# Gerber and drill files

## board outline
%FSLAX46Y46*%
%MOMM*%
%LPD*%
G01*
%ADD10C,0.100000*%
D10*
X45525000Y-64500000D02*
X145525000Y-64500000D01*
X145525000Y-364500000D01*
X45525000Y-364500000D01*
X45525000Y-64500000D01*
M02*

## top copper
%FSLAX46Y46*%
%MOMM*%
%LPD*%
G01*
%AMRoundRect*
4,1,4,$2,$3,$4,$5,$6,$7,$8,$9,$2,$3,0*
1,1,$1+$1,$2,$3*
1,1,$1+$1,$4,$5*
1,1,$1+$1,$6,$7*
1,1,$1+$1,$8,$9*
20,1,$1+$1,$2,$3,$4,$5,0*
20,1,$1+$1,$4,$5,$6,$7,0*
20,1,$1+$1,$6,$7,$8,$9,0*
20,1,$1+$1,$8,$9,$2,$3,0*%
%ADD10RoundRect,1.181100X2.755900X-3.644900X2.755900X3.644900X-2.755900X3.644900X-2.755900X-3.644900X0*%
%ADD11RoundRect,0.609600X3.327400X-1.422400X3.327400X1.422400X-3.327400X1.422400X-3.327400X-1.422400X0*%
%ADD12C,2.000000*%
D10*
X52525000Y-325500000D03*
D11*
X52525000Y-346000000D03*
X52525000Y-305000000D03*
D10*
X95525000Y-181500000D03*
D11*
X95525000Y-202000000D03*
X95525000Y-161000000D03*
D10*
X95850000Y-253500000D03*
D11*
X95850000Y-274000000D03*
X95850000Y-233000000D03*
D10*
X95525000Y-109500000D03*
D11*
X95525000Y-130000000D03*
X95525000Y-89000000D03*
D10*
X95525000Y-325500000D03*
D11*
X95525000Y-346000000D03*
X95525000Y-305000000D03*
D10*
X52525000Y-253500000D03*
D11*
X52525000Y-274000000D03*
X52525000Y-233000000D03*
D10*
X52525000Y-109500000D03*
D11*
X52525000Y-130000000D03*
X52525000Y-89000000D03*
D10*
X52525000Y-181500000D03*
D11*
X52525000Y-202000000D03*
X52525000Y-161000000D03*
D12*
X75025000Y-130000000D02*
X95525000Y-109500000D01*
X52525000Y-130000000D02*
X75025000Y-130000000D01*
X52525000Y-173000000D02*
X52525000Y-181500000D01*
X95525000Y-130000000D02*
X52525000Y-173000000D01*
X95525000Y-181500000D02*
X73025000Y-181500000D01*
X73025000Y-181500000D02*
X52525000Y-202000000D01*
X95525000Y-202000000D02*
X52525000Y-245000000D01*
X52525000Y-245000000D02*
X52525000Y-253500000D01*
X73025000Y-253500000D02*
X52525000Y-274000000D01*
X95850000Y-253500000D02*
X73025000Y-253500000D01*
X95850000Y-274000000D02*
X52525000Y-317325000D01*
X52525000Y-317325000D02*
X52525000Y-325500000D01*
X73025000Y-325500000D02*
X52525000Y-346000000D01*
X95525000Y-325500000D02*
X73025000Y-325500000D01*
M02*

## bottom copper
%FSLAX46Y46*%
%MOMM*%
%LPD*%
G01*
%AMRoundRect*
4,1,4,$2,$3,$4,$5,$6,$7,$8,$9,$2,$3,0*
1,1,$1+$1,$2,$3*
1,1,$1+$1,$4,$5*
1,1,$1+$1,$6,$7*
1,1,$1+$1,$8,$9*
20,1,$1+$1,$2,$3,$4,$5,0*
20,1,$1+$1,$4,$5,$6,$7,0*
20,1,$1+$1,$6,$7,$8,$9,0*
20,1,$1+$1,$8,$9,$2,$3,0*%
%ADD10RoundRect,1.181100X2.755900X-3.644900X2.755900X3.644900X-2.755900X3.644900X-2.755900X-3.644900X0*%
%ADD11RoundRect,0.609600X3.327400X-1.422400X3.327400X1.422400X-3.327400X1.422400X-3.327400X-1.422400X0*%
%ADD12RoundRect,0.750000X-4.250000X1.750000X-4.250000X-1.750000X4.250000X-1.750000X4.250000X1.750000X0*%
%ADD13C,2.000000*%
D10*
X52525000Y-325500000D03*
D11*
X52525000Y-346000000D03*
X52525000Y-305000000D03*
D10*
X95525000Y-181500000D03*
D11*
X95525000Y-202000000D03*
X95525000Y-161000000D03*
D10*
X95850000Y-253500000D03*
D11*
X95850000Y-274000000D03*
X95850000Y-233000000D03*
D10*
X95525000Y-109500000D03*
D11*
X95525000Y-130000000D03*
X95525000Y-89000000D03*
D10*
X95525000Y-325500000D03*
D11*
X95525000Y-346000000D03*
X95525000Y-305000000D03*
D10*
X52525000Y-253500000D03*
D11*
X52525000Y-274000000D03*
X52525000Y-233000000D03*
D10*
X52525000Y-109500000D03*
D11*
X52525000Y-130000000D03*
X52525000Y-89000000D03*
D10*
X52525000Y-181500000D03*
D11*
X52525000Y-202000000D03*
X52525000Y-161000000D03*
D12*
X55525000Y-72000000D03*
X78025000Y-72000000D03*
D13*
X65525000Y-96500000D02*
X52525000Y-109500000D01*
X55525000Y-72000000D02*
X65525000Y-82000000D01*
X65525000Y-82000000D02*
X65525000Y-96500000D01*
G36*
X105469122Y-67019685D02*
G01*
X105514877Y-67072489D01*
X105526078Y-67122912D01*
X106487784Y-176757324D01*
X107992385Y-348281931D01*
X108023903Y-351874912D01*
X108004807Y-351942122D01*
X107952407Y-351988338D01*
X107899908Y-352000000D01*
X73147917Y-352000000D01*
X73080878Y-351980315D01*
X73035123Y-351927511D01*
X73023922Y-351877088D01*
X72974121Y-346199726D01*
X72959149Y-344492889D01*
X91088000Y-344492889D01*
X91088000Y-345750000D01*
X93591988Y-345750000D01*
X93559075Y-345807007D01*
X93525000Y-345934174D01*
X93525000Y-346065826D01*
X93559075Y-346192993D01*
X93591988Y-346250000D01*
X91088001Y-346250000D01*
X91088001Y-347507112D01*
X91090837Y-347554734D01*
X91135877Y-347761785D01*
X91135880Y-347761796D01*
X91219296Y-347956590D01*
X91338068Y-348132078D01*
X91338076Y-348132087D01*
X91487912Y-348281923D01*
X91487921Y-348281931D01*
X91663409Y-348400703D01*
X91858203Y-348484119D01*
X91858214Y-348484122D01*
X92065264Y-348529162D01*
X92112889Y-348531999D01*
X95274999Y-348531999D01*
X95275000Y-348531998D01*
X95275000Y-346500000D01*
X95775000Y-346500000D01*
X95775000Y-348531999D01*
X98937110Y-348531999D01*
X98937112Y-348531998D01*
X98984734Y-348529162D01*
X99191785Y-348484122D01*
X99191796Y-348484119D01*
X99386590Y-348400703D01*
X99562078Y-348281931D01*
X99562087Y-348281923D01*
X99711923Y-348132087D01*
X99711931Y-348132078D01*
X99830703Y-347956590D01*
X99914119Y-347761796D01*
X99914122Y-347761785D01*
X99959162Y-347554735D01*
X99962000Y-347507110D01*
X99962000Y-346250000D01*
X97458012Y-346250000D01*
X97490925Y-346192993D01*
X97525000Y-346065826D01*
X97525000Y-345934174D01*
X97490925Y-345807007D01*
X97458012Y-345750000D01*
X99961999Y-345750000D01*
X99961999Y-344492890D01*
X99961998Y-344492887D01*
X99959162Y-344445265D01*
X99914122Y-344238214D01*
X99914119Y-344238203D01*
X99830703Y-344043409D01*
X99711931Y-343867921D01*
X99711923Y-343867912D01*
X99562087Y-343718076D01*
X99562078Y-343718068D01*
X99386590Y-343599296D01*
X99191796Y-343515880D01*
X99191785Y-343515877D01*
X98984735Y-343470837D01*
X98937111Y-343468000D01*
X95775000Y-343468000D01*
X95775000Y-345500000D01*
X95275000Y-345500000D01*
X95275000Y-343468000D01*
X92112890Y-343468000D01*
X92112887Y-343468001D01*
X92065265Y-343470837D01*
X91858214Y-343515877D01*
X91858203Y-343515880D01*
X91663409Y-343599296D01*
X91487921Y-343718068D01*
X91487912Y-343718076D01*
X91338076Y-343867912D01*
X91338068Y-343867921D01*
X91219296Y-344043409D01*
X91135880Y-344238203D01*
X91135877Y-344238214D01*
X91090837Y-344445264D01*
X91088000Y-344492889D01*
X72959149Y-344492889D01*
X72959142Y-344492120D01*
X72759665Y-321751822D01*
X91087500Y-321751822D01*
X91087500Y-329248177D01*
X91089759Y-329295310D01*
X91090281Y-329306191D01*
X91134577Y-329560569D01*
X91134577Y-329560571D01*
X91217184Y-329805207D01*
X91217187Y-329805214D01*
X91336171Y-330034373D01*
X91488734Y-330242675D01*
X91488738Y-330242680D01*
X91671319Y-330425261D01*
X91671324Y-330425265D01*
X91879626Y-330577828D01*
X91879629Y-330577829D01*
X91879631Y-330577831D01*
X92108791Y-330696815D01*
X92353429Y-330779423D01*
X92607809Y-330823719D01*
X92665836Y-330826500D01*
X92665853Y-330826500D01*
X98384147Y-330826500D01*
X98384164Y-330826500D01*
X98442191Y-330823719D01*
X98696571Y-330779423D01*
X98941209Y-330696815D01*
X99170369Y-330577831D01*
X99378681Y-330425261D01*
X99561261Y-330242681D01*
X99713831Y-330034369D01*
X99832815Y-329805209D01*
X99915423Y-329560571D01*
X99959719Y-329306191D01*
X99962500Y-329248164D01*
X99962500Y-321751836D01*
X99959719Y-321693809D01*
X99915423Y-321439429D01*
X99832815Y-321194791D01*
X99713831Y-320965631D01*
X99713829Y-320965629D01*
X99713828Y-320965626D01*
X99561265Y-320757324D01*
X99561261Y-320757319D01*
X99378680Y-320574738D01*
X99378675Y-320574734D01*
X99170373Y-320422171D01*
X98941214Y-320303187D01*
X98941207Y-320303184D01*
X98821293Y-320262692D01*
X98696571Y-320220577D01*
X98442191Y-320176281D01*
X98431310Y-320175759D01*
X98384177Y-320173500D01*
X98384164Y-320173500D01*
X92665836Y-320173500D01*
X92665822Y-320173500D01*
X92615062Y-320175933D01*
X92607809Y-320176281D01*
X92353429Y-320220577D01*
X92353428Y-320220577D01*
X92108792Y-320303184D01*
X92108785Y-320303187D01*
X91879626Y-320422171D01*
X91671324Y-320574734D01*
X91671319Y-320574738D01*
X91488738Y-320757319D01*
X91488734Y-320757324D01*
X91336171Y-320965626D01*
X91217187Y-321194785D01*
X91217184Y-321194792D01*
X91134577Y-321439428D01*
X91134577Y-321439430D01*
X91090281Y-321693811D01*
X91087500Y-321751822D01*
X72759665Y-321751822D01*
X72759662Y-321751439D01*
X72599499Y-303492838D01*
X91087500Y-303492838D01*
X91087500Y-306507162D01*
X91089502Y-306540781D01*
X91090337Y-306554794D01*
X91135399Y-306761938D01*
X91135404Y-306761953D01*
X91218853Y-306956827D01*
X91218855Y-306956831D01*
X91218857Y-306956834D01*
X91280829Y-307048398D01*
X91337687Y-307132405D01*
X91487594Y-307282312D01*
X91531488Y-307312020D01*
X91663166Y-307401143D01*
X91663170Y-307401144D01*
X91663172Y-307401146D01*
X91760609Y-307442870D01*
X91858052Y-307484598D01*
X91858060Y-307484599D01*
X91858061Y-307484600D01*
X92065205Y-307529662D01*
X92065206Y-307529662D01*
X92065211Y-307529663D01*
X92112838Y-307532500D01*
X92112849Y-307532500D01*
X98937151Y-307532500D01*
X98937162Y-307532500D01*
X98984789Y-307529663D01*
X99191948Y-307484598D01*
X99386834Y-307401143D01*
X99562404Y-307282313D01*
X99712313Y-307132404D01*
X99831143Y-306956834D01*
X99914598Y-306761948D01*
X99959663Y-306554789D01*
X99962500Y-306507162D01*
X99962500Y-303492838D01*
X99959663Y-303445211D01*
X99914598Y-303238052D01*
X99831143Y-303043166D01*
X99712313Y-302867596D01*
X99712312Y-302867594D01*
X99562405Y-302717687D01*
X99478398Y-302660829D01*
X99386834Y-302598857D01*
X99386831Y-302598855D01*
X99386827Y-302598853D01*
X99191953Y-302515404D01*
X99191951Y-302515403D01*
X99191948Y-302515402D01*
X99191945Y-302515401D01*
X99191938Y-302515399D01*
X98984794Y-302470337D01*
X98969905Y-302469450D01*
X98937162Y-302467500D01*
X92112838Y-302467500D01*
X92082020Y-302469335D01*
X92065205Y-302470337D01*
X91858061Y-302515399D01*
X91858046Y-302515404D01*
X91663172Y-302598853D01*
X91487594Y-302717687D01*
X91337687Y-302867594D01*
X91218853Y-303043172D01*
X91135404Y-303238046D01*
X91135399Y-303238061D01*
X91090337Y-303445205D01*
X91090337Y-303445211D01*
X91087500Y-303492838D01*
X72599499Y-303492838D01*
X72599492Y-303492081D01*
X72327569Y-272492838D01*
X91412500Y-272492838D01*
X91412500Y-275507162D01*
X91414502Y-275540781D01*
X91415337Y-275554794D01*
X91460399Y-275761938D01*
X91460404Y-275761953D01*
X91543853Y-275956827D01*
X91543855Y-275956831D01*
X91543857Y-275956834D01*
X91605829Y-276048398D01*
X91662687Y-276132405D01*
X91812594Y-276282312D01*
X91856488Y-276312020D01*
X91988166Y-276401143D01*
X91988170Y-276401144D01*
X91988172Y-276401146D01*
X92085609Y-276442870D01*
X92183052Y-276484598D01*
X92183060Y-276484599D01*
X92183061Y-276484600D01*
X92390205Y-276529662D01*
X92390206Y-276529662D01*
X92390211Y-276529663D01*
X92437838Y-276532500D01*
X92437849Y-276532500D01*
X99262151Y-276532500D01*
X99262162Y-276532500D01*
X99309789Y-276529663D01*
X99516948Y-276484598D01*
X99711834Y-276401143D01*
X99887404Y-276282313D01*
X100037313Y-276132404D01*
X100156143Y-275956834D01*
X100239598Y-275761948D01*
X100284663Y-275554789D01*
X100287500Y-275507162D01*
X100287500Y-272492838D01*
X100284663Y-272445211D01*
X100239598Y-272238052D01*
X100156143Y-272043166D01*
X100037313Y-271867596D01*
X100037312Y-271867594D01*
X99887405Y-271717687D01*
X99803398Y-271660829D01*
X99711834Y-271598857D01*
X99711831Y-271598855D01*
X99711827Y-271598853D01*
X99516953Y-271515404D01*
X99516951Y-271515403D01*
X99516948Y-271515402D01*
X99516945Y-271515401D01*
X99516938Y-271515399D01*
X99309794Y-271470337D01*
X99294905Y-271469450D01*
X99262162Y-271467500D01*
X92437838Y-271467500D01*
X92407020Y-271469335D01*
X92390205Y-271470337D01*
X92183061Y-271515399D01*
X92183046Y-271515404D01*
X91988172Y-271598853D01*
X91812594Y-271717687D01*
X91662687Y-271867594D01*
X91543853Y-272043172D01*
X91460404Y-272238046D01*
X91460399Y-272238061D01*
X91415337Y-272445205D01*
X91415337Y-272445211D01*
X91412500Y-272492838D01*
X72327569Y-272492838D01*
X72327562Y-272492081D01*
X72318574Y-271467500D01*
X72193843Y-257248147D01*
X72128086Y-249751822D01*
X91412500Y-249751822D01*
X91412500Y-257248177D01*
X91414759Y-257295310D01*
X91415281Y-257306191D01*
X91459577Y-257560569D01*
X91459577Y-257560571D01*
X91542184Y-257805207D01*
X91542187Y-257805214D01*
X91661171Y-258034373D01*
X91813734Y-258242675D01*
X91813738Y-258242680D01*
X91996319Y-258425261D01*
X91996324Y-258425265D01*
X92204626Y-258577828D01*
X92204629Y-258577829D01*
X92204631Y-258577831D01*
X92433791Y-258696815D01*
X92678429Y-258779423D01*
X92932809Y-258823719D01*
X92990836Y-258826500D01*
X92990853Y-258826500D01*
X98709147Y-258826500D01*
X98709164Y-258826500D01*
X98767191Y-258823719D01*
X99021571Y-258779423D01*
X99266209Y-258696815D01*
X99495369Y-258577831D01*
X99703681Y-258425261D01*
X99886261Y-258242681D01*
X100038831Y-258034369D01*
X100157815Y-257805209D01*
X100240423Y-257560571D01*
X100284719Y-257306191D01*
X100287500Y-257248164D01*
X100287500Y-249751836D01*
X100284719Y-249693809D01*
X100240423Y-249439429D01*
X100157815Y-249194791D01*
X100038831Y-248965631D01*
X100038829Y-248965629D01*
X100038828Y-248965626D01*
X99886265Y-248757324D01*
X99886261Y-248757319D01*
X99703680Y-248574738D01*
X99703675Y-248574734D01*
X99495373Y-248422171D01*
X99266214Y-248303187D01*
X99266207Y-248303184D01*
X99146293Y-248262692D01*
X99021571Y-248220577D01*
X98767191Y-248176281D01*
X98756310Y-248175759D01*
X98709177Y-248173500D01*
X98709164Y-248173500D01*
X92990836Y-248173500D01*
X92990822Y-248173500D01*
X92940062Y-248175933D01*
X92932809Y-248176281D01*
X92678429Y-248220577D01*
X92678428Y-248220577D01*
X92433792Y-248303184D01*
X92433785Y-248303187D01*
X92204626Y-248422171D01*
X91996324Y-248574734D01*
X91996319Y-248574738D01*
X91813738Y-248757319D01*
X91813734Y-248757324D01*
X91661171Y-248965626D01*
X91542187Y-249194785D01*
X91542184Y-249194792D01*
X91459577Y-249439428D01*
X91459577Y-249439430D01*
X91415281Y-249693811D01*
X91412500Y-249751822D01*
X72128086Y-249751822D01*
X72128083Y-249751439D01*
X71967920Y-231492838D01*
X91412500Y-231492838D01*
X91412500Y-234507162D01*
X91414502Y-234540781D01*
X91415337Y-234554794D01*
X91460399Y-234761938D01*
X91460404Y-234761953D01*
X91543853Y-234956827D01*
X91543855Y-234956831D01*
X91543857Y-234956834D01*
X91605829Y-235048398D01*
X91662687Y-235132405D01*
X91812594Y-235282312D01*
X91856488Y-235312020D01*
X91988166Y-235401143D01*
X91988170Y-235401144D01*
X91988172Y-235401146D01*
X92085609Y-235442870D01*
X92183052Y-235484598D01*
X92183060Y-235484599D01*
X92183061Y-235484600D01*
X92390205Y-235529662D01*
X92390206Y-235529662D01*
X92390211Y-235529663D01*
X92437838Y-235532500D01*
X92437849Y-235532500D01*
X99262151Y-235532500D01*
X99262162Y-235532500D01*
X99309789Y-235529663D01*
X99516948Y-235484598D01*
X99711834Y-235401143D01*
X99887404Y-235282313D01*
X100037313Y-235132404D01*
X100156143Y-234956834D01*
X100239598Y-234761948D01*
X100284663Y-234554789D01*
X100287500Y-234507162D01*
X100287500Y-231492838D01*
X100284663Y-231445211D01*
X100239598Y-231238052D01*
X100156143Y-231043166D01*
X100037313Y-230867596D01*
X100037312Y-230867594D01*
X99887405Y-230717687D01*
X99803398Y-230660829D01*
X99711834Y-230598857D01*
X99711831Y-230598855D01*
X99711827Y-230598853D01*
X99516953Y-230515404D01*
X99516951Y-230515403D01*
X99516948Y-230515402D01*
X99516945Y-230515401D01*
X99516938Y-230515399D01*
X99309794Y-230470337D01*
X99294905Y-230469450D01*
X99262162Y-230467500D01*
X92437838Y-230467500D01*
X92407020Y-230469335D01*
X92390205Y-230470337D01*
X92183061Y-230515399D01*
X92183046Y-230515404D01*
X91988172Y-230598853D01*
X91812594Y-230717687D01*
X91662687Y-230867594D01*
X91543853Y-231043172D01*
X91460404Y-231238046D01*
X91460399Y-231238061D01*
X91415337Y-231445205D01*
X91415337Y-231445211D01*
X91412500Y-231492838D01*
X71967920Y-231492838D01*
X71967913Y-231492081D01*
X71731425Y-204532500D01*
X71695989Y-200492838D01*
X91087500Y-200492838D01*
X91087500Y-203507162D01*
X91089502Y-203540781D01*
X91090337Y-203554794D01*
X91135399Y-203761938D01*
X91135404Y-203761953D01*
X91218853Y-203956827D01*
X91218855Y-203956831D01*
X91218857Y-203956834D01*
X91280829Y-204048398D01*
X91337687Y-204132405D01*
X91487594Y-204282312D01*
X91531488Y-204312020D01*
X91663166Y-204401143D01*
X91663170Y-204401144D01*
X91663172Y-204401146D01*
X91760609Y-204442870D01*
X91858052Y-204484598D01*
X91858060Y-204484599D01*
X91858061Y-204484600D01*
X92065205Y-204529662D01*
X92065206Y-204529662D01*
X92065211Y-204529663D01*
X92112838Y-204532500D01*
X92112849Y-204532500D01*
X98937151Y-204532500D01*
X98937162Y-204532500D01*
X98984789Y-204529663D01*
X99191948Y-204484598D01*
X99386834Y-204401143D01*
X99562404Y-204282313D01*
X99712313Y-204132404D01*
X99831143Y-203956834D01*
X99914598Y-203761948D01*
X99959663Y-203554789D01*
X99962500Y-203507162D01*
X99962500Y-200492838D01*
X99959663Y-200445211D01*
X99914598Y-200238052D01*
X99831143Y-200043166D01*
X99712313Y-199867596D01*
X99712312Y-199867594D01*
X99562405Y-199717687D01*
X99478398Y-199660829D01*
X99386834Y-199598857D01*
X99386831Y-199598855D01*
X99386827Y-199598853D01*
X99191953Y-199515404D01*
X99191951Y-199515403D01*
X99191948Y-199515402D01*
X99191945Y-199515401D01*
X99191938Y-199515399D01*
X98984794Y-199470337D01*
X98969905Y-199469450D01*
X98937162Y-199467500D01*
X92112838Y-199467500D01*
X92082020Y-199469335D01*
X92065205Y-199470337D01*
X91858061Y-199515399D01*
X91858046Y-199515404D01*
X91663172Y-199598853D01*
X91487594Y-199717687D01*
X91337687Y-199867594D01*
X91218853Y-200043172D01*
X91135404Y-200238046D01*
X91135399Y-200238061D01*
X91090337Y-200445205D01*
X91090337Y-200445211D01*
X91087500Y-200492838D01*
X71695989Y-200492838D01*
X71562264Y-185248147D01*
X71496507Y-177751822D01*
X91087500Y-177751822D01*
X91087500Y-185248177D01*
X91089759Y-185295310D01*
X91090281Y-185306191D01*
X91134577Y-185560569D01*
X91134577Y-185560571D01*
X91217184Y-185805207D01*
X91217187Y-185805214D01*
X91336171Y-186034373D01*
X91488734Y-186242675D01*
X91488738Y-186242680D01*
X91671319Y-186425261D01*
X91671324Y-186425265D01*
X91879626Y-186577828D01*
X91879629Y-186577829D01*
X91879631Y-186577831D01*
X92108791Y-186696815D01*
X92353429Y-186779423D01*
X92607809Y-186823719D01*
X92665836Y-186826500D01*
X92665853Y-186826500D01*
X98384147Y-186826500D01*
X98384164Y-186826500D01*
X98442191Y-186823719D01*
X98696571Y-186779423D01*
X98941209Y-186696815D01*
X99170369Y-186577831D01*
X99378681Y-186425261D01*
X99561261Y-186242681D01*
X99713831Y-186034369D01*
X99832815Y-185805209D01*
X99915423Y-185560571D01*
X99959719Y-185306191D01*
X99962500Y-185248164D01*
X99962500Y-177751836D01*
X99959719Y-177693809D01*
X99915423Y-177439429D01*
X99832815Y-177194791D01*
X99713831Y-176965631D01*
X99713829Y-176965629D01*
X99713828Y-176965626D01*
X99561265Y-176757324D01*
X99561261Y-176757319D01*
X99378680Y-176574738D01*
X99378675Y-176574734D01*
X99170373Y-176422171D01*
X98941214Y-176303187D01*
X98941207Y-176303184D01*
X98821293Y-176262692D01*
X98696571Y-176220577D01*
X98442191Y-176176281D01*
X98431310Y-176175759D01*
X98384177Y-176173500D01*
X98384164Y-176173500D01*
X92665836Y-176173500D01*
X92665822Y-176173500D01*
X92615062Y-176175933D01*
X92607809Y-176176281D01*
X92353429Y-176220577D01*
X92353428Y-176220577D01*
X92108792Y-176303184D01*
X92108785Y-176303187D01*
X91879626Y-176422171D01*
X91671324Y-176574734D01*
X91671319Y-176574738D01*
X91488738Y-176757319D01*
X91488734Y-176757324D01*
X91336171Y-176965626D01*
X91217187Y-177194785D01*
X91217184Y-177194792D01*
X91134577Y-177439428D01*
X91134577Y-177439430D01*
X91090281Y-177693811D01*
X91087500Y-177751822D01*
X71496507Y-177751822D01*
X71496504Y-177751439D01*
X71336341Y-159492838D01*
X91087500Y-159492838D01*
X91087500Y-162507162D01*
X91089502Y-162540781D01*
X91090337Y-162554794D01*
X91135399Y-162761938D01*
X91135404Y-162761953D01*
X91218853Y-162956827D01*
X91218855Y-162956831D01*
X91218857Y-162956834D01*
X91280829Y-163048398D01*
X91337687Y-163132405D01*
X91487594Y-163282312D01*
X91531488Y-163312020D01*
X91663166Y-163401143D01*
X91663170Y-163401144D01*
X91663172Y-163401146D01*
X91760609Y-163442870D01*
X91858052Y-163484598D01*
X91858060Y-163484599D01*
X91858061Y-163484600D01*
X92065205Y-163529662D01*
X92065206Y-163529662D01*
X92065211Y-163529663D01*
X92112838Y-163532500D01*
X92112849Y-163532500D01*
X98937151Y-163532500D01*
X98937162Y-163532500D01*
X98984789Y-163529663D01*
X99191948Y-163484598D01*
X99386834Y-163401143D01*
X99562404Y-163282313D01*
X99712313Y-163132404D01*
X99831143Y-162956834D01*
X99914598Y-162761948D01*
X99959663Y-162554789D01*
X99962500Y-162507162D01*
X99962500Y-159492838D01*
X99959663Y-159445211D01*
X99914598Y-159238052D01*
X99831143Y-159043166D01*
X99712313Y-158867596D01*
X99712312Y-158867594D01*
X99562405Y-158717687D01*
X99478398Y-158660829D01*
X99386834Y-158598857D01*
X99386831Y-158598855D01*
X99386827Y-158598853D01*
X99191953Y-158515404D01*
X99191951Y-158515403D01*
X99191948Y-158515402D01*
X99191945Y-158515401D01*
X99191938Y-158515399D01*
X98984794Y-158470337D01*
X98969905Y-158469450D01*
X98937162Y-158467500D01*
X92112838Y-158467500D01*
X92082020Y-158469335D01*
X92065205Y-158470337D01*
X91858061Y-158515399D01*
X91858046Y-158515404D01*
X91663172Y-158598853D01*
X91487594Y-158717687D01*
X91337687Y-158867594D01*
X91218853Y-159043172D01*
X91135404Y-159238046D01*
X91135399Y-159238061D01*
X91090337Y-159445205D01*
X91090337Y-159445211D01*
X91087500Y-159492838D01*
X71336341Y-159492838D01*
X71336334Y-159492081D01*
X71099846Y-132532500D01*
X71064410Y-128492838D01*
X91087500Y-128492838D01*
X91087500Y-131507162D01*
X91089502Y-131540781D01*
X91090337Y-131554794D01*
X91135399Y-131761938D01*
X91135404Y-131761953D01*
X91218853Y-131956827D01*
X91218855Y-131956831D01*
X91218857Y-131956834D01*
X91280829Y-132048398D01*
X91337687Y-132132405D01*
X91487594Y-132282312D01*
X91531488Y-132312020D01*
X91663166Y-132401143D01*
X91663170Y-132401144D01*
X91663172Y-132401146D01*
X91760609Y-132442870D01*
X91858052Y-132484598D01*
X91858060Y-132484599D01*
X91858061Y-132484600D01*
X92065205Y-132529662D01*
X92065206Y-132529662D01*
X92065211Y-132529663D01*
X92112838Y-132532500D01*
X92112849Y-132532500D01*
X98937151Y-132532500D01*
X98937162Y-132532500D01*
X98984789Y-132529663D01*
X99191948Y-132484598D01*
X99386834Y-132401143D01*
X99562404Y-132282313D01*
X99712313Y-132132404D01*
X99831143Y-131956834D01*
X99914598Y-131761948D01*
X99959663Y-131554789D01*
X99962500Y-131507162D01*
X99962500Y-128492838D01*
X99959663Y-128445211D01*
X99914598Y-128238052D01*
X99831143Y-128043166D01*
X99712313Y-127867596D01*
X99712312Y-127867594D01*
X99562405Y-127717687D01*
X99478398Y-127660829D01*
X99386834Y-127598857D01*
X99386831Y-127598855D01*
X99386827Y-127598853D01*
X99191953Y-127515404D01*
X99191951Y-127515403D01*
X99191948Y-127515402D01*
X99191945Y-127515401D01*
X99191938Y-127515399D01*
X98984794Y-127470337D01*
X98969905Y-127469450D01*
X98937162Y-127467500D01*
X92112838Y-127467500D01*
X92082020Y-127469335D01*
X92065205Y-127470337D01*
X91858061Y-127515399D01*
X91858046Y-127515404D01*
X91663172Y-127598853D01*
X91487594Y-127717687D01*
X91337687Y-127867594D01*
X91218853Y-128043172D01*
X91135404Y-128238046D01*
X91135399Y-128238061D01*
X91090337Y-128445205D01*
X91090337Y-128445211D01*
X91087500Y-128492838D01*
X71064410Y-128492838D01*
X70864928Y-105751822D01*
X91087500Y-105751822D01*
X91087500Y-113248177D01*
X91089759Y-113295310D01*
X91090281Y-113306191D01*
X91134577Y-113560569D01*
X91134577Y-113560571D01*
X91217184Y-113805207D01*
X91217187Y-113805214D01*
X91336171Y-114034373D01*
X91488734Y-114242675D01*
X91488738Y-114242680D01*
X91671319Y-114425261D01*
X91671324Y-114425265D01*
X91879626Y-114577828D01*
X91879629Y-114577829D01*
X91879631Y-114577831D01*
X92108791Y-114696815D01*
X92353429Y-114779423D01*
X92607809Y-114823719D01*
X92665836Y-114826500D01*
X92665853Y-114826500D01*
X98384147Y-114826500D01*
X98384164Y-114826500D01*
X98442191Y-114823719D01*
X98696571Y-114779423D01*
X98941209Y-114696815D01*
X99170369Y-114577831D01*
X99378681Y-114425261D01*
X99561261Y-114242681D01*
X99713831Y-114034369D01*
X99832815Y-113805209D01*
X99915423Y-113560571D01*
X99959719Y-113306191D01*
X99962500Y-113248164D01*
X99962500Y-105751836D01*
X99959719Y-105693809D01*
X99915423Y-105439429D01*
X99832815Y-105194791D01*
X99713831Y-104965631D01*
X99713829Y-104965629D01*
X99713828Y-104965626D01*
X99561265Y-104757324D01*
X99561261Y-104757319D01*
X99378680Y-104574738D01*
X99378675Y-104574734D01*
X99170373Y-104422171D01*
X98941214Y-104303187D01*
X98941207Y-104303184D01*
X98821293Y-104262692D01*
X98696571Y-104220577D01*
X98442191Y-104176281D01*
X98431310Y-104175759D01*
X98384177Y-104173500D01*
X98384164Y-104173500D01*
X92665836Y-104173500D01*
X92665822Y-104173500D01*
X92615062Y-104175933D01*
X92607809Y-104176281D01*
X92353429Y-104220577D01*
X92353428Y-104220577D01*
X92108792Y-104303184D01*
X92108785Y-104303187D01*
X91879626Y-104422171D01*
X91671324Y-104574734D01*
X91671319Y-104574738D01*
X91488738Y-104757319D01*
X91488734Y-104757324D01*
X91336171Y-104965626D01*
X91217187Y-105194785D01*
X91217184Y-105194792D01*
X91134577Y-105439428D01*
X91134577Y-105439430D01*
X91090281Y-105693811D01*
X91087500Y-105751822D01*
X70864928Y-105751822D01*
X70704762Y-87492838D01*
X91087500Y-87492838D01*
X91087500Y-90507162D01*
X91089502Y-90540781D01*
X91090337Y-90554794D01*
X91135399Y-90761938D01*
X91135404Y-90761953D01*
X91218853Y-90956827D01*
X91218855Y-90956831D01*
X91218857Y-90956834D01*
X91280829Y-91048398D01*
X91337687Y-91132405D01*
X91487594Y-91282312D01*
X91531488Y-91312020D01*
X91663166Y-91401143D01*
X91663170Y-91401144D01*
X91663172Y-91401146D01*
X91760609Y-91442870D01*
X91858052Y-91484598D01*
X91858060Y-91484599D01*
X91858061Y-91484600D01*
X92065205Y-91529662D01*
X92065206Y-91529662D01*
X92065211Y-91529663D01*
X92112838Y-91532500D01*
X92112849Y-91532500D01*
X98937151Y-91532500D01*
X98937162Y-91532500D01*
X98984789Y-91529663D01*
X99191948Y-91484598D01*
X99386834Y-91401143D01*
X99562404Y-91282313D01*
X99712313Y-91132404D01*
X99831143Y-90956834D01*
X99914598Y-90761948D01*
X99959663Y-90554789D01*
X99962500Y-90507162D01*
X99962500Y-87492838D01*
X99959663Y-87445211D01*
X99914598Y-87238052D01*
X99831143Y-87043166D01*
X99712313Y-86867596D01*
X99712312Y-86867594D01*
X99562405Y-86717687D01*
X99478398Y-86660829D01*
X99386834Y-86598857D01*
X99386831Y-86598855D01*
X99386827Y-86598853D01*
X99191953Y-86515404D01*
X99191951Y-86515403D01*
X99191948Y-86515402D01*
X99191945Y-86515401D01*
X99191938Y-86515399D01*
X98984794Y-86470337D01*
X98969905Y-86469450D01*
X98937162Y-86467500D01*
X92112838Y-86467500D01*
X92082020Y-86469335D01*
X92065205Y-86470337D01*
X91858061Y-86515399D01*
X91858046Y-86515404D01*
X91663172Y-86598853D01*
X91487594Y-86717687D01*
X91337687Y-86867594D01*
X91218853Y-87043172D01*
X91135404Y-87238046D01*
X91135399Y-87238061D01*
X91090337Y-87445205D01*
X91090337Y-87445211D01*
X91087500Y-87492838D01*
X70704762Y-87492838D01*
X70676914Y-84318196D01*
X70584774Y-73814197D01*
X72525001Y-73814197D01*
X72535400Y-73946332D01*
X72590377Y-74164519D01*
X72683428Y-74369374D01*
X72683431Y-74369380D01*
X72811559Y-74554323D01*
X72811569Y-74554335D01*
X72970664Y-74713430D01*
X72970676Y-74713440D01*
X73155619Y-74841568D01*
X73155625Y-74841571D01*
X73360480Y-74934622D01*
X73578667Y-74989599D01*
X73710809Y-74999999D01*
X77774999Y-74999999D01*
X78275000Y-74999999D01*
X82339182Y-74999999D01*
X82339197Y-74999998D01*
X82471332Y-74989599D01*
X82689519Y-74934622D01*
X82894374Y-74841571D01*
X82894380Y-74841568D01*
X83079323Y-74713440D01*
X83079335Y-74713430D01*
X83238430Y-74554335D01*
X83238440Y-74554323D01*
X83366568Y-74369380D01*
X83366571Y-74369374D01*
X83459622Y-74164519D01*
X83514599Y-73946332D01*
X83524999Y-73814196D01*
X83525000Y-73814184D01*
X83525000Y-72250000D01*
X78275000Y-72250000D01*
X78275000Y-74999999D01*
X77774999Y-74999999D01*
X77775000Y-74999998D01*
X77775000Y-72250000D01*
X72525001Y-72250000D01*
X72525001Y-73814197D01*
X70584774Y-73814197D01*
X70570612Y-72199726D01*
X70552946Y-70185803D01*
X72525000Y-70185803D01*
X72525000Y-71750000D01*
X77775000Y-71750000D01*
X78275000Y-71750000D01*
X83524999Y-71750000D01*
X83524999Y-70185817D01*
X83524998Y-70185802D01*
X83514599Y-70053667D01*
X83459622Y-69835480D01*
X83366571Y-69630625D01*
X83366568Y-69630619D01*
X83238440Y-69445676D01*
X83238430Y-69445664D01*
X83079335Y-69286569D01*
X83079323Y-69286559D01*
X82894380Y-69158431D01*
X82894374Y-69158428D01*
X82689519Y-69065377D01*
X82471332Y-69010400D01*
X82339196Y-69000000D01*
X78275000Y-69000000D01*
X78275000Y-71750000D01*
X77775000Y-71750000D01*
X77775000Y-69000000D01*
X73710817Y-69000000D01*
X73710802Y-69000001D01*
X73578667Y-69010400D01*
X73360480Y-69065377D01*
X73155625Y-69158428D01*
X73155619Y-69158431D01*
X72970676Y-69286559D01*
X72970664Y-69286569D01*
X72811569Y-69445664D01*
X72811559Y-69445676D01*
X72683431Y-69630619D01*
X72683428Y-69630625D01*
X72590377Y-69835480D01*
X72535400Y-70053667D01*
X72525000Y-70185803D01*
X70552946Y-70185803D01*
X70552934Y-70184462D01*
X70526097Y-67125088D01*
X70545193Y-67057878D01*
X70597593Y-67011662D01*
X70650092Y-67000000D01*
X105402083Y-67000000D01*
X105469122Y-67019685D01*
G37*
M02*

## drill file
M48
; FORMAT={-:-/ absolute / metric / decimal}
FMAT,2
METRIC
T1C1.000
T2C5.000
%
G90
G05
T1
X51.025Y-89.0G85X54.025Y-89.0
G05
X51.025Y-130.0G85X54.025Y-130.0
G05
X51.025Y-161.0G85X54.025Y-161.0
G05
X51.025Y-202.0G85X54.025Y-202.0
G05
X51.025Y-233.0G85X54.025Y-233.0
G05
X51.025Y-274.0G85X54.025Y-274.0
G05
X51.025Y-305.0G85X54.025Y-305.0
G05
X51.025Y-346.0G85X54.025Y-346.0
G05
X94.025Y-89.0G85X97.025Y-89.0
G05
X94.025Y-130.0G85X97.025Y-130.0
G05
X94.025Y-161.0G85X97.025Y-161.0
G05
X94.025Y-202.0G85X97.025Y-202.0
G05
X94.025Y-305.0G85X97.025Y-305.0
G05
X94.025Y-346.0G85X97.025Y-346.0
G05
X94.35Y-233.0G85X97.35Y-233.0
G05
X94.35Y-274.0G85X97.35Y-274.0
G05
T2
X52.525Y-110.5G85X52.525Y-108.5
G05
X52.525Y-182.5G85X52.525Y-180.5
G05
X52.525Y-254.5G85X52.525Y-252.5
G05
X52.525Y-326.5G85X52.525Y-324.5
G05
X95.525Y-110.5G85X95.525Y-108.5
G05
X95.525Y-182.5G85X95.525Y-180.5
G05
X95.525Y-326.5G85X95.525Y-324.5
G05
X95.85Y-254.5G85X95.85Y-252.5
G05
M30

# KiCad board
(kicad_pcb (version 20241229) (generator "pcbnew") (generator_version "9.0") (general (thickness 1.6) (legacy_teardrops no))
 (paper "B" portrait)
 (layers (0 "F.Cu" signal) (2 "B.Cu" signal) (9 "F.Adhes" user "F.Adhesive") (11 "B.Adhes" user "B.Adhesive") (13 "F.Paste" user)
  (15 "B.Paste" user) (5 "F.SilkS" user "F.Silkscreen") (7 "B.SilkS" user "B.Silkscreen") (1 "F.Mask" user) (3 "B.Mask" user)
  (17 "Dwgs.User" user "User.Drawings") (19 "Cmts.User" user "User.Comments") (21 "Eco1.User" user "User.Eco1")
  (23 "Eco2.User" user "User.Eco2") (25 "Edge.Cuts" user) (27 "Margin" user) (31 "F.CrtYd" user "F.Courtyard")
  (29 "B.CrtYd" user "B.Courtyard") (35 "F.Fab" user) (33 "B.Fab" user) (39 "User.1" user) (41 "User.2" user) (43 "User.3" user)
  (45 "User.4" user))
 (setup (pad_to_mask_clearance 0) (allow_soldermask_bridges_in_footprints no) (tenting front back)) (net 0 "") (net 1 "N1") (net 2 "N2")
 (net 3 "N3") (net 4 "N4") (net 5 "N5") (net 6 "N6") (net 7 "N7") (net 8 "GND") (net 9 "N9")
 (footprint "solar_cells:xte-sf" (layer "F.Cu") (at 76.525 325.5 90)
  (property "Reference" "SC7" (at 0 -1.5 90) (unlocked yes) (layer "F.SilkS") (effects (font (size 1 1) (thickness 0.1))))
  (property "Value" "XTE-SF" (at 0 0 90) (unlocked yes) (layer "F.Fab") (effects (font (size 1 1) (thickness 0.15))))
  (pad "1" thru_hole roundrect (at 0 -24 90) (size 9.652 7.874) (drill oval 7 5) (layers "*.Cu" "*.Mask") (remove_unused_layers no)
   (roundrect_rratio 0.15) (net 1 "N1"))
  (pad "2" thru_hole roundrect (at -20.5 -24 90) (size 4.064 7.874) (drill oval 1 4) (layers "*.Cu" "*.Mask") (remove_unused_layers no)
   (roundrect_rratio 0.15) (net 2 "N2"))
  (pad "3" thru_hole roundrect (at 20.5 -24 90) (size 4.064 7.874) (drill oval 1 4) (layers "*.Cu" "*.Mask") (remove_unused_layers no)
   (roundrect_rratio 0.15)))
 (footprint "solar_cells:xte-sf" (layer "F.Cu") (at 119.525 181.5 90)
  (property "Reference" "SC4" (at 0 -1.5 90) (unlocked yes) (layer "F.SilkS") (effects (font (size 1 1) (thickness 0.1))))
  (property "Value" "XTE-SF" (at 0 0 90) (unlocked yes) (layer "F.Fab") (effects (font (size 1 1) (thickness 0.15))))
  (pad "1" thru_hole roundrect (at 0 -24 90) (size 9.652 7.874) (drill oval 7 5) (layers "*.Cu" "*.Mask") (remove_unused_layers no)
   (roundrect_rratio 0.15) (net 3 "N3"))
  (pad "2" thru_hole roundrect (at -20.5 -24 90) (size 4.064 7.874) (drill oval 1 4) (layers "*.Cu" "*.Mask") (remove_unused_layers no)
   (roundrect_rratio 0.15) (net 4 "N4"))
  (pad "3" thru_hole roundrect (at 20.5 -24 90) (size 4.064 7.874) (drill oval 1 4) (layers "*.Cu" "*.Mask") (remove_unused_layers no)
   (roundrect_rratio 0.15)))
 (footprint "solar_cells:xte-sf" (layer "F.Cu") (at 119.85 253.5 90)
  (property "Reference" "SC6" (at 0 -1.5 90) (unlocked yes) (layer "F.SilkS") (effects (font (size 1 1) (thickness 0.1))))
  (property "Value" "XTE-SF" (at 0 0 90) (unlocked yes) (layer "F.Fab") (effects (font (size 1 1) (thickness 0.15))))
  (pad "1" thru_hole roundrect (at 0 -24 90) (size 9.652 7.874) (drill oval 7 5) (layers "*.Cu" "*.Mask") (remove_unused_layers no)
   (roundrect_rratio 0.15) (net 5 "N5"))
  (pad "2" thru_hole roundrect (at -20.5 -24 90) (size 4.064 7.874) (drill oval 1 4) (layers "*.Cu" "*.Mask") (remove_unused_layers no)
   (roundrect_rratio 0.15) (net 1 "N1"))
  (pad "3" thru_hole roundrect (at 20.5 -24 90) (size 4.064 7.874) (drill oval 1 4) (layers "*.Cu" "*.Mask") (remove_unused_layers no)
   (roundrect_rratio 0.15)))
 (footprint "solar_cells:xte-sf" (layer "F.Cu") (at 119.525 109.5 90)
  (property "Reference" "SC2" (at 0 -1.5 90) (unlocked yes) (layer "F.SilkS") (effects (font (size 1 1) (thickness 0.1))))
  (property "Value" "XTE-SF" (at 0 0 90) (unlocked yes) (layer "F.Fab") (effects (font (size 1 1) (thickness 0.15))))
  (pad "1" thru_hole roundrect (at 0 -24 90) (size 9.652 7.874) (drill oval 7 5) (layers "*.Cu" "*.Mask") (remove_unused_layers no)
   (roundrect_rratio 0.15) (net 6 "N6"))
  (pad "2" thru_hole roundrect (at -20.5 -24 90) (size 4.064 7.874) (drill oval 1 4) (layers "*.Cu" "*.Mask") (remove_unused_layers no)
   (roundrect_rratio 0.15) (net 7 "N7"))
  (pad "3" thru_hole roundrect (at 20.5 -24 90) (size 4.064 7.874) (drill oval 1 4) (layers "*.Cu" "*.Mask") (remove_unused_layers no)
   (roundrect_rratio 0.15)))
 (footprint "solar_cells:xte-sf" (layer "F.Cu") (at 119.525 325.5 90)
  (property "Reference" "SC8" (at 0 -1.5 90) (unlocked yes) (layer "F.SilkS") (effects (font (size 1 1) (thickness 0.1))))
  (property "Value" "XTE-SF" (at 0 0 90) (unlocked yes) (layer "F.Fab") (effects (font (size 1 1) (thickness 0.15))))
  (pad "1" thru_hole roundrect (at 0 -24 90) (size 9.652 7.874) (drill oval 7 5) (layers "*.Cu" "*.Mask") (remove_unused_layers no)
   (roundrect_rratio 0.15) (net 2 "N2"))
  (pad "2" thru_hole roundrect (at -20.5 -24 90) (size 4.064 7.874) (drill oval 1 4) (layers "*.Cu" "*.Mask") (remove_unused_layers no)
   (roundrect_rratio 0.15) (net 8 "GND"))
  (pad "3" thru_hole roundrect (at 20.5 -24 90) (size 4.064 7.874) (drill oval 1 4) (layers "*.Cu" "*.Mask") (remove_unused_layers no)
   (roundrect_rratio 0.15)))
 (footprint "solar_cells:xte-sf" (layer "F.Cu") (at 76.525 253.5 90)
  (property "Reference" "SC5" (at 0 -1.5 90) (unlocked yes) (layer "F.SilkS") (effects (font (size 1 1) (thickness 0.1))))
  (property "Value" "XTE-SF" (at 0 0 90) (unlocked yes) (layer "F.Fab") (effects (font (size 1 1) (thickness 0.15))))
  (pad "1" thru_hole roundrect (at 0 -24 90) (size 9.652 7.874) (drill oval 7 5) (layers "*.Cu" "*.Mask") (remove_unused_layers no)
   (roundrect_rratio 0.15) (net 4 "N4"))
  (pad "2" thru_hole roundrect (at -20.5 -24 90) (size 4.064 7.874) (drill oval 1 4) (layers "*.Cu" "*.Mask") (remove_unused_layers no)
   (roundrect_rratio 0.15) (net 5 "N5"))
  (pad "3" thru_hole roundrect (at 20.5 -24 90) (size 4.064 7.874) (drill oval 1 4) (layers "*.Cu" "*.Mask") (remove_unused_layers no)
   (roundrect_rratio 0.15)))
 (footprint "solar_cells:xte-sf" (layer "F.Cu") (at 76.525 109.5 90)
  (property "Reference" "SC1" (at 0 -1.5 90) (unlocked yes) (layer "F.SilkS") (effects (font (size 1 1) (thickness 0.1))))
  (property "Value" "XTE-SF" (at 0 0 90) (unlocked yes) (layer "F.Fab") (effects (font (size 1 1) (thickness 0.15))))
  (pad "1" thru_hole roundrect (at 0 -24 90) (size 9.652 7.874) (drill oval 7 5) (layers "*.Cu" "*.Mask") (remove_unused_layers no)
   (roundrect_rratio 0.15) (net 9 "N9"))
  (pad "2" thru_hole roundrect (at -20.5 -24 90) (size 4.064 7.874) (drill oval 1 4) (layers "*.Cu" "*.Mask") (remove_unused_layers no)
   (roundrect_rratio 0.15) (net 6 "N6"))
  (pad "3" thru_hole roundrect (at 20.5 -24 90) (size 4.064 7.874) (drill oval 1 4) (layers "*.Cu" "*.Mask") (remove_unused_layers no)
   (roundrect_rratio 0.15)))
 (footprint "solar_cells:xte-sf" (layer "F.Cu") (at 76.525 181.5 90)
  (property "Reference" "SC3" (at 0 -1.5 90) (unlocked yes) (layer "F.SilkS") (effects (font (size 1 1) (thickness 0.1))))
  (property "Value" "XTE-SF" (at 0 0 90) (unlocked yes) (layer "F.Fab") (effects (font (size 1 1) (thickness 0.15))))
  (pad "1" thru_hole roundrect (at 0 -24 90) (size 9.652 7.874) (drill oval 7 5) (layers "*.Cu" "*.Mask") (remove_unused_layers no)
   (roundrect_rratio 0.15) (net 7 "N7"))
  (pad "2" thru_hole roundrect (at -20.5 -24 90) (size 4.064 7.874) (drill oval 1 4) (layers "*.Cu" "*.Mask") (remove_unused_layers no)
   (roundrect_rratio 0.15) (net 3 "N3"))
  (pad "3" thru_hole roundrect (at 20.5 -24 90) (size 4.064 7.874) (drill oval 1 4) (layers "*.Cu" "*.Mask") (remove_unused_layers no)
   (roundrect_rratio 0.15)))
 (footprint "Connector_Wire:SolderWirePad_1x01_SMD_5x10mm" (layer "B.Cu") (at 55.525 72 -90)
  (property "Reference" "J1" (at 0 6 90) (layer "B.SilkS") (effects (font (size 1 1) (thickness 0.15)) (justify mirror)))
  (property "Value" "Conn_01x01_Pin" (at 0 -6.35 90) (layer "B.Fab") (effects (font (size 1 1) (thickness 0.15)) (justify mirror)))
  (pad "1" smd roundrect (at 0 0 270) (size 5 10) (layers "F.Mask" "B.Cu" "F.Paste") (roundrect_rratio 0.15) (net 9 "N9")))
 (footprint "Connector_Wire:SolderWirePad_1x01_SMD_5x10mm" (layer "B.Cu") (at 78.025 72 -90)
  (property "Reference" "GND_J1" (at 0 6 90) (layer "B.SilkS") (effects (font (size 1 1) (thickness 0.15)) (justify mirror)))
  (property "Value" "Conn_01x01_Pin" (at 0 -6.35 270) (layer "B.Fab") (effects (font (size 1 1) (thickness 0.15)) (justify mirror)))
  (pad "1" smd roundrect (at 0 0 270) (size 5 10) (layers "F.Mask" "B.Cu" "F.Paste") (roundrect_rratio 0.15) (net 8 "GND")))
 (gr_rect (start 45.525 64.5) (end 145.525 364.5) (stroke (width 0.1) (type solid)) (fill no) (layer "Edge.Cuts"))
 (segment (start 65.525 96.5) (end 52.525 109.5) (width 2) (layer "B.Cu") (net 9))
 (segment (start 55.525 72) (end 65.525 82) (width 2) (layer "B.Cu") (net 9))
 (segment (start 65.525 82) (end 65.525 96.5) (width 2) (layer "B.Cu") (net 9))
 (segment (start 75.025 130) (end 95.525 109.5) (width 2) (layer "F.Cu") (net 6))
 (segment (start 52.525 130) (end 75.025 130) (width 2) (layer "F.Cu") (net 6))
 (segment (start 52.525 173) (end 52.525 181.5) (width 2) (layer "F.Cu") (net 7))
 (segment (start 95.525 130) (end 52.525 173) (width 2) (layer "F.Cu") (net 7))
 (segment (start 95.525 181.5) (end 73.025 181.5) (width 2) (layer "F.Cu") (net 3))
 (segment (start 73.025 181.5) (end 52.525 202) (width 2) (layer "F.Cu") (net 3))
 (segment (start 95.525 202) (end 52.525 245) (width 2) (layer "F.Cu") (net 4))
 (segment (start 52.525 245) (end 52.525 253.5) (width 2) (layer "F.Cu") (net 4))
 (segment (start 73.025 253.5) (end 52.525 274) (width 2) (layer "F.Cu") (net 5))
 (segment (start 95.85 253.5) (end 73.025 253.5) (width 2) (layer "F.Cu") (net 5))
 (segment (start 95.85 274) (end 52.525 317.325) (width 2) (layer "F.Cu") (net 1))
 (segment (start 52.525 317.325) (end 52.525 325.5) (width 2) (layer "F.Cu") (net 1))
 (segment (start 73.025 325.5) (end 52.525 346) (width 2) (layer "F.Cu") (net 2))
 (segment (start 95.525 325.5) (end 73.025 325.5) (width 2) (layer "F.Cu") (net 2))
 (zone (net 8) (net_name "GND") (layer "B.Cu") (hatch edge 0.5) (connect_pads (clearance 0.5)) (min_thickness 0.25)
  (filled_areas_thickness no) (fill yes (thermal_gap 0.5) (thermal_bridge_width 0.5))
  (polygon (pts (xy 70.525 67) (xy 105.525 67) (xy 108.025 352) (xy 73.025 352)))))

